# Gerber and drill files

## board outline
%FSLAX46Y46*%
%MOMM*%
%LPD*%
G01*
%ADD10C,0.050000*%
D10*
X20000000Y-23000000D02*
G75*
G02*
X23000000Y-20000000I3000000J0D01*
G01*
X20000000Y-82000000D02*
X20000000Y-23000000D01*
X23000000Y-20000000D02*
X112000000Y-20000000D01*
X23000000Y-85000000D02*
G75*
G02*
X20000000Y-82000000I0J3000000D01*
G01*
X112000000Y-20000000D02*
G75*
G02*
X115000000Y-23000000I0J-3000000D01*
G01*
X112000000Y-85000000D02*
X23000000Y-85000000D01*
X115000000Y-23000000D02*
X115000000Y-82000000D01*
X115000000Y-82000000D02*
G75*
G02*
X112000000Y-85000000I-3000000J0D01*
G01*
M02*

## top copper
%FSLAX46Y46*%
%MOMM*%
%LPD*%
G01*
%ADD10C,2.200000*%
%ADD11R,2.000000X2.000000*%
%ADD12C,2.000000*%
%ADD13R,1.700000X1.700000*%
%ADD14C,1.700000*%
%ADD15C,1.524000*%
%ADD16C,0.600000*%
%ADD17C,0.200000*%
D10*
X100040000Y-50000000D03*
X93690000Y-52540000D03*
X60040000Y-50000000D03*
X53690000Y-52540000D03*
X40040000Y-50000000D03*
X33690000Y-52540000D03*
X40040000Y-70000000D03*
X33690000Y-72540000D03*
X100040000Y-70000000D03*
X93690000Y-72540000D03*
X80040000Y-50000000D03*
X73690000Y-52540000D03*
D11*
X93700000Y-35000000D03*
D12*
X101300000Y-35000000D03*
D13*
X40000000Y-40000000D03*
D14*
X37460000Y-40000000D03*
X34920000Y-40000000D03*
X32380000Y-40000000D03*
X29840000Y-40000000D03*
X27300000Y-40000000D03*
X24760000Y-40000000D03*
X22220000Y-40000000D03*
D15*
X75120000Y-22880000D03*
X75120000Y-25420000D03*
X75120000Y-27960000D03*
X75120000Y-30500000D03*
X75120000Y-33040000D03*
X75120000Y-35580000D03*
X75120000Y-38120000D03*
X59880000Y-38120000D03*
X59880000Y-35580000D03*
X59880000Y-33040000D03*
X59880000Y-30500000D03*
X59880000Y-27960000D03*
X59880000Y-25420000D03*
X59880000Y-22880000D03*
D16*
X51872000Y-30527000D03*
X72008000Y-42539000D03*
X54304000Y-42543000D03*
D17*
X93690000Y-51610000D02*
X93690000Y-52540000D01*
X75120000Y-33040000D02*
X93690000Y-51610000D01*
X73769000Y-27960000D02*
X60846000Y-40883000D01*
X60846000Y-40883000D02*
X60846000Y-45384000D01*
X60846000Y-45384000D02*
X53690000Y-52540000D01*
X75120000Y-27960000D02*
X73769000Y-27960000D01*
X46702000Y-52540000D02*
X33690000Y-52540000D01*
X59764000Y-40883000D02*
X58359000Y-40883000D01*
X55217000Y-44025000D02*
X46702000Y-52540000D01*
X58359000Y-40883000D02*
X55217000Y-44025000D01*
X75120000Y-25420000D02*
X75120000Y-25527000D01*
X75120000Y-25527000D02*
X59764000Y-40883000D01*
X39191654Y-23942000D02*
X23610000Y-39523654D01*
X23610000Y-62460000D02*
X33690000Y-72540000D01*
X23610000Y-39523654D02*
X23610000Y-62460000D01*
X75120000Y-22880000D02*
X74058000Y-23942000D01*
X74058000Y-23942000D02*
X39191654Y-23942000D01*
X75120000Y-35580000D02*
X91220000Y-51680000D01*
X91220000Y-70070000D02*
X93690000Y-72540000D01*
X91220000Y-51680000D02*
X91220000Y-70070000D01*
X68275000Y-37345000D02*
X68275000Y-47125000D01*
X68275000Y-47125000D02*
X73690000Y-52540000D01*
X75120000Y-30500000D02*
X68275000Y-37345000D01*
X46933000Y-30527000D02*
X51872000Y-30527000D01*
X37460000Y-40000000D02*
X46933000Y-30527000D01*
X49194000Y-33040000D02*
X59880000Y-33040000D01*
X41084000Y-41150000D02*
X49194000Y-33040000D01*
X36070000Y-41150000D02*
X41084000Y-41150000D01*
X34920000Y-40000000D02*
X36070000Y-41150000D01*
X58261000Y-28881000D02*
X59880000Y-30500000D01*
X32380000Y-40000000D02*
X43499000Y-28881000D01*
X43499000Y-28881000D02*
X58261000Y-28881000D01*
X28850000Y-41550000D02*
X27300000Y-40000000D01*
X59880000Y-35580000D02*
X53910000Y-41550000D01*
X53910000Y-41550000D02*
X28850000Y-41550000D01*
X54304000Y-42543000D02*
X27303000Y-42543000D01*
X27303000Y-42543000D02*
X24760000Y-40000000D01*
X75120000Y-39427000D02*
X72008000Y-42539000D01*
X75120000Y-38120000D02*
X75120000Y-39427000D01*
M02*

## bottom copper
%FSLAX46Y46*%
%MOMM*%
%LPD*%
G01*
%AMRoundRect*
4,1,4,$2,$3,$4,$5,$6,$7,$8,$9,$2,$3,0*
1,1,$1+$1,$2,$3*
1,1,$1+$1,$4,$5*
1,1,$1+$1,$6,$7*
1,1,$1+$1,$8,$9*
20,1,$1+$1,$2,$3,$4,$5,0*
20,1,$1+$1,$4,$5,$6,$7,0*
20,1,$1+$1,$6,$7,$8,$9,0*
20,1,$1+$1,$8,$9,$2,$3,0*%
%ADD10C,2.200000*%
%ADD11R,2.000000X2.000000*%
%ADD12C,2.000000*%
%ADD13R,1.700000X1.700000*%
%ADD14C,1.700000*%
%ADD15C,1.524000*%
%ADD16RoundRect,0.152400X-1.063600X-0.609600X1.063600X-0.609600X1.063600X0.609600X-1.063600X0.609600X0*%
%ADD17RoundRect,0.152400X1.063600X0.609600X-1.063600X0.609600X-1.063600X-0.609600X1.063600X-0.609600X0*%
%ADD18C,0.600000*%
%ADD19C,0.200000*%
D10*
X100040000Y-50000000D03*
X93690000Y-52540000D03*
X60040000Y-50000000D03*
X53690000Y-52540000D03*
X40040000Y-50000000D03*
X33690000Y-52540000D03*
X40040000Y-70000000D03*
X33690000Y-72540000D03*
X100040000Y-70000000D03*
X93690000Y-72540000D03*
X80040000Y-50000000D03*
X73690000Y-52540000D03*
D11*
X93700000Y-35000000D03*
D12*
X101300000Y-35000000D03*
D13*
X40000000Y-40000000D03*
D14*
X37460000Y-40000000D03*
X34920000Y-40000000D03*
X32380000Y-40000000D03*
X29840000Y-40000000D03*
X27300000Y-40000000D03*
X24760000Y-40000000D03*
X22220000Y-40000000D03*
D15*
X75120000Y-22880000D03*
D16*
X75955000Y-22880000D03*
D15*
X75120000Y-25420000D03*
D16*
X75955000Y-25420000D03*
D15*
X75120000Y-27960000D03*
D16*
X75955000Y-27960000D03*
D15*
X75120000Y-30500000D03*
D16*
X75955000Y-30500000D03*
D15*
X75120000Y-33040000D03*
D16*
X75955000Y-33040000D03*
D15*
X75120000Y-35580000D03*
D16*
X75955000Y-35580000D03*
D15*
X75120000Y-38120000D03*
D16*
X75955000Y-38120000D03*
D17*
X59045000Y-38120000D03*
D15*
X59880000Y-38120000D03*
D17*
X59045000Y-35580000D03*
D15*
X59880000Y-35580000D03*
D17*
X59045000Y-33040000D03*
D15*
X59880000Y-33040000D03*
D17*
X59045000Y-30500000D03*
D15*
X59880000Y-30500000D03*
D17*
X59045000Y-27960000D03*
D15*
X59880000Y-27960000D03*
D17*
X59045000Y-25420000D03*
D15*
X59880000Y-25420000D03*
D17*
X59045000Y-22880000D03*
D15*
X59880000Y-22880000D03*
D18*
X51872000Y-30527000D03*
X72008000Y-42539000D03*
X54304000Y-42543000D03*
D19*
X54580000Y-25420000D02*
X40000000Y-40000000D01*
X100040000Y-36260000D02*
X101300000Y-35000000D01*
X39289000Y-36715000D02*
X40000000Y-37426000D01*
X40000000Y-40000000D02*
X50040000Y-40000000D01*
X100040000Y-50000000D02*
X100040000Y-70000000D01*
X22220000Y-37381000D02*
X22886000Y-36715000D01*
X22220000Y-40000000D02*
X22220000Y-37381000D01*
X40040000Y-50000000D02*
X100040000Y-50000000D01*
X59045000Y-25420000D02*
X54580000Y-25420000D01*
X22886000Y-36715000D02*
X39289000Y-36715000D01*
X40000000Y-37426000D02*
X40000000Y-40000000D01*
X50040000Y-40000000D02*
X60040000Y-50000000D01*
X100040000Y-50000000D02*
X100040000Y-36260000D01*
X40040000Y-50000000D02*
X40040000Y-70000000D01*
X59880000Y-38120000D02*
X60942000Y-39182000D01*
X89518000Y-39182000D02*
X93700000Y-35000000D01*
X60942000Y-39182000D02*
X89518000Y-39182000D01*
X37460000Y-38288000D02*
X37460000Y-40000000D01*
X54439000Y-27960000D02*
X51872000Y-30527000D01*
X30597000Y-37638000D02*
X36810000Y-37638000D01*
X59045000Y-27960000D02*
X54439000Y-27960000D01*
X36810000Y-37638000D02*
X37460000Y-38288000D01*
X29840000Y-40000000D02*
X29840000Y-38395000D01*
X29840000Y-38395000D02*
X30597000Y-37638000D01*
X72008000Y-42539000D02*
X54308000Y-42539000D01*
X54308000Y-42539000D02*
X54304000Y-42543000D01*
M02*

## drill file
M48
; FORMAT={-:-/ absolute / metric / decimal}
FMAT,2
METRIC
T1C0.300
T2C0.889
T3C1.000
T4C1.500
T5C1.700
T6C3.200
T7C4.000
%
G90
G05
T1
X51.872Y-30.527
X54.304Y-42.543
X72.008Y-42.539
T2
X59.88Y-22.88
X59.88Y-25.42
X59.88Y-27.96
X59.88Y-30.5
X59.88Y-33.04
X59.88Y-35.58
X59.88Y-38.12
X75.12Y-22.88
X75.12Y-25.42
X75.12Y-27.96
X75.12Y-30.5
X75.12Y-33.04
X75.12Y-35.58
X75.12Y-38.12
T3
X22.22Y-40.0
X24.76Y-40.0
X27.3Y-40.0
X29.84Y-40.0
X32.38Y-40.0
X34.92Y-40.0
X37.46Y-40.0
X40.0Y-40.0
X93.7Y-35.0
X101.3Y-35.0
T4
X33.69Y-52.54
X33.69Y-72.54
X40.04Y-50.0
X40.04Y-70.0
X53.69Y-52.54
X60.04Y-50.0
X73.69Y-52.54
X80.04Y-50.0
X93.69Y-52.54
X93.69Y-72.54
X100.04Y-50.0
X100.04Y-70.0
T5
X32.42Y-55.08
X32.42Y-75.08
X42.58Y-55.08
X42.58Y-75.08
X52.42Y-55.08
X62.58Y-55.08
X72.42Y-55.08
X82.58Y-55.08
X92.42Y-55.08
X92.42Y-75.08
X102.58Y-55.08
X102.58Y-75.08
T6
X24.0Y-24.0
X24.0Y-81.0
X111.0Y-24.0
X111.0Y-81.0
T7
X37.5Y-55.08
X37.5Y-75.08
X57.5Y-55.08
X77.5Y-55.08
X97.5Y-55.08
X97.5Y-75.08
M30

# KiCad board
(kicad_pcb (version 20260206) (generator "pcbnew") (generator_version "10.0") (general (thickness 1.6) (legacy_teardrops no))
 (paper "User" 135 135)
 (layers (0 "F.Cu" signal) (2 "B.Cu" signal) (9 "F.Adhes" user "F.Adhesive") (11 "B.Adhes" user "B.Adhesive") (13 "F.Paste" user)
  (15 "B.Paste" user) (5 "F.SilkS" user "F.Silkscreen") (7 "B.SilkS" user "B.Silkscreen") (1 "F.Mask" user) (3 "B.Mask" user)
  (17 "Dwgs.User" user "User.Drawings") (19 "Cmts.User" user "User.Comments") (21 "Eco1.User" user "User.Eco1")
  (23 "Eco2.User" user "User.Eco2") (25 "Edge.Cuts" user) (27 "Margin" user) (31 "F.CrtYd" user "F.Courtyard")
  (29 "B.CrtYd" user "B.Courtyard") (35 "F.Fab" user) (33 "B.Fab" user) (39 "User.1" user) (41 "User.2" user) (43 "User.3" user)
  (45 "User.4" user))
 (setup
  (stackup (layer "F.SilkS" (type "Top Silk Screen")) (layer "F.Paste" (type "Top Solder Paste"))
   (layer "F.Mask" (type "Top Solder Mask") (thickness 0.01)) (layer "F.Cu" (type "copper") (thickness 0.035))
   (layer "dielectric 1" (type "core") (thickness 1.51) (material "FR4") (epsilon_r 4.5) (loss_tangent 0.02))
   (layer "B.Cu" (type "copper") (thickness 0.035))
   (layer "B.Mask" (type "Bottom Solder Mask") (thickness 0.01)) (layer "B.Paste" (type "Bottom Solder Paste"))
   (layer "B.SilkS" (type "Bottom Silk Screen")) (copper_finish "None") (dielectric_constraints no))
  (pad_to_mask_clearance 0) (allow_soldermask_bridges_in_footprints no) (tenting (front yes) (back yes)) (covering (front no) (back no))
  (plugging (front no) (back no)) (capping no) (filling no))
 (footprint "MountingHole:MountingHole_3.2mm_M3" (layer "F.Cu") (at 24 81)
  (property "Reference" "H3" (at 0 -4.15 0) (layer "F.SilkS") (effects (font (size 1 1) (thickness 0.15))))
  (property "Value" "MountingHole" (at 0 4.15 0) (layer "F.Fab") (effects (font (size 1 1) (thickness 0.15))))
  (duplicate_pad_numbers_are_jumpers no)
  (pad "" np_thru_hole circle (at 0 0) (size 3.2 3.2) (drill 3.2) (layers "*.Cu" "*.Mask")))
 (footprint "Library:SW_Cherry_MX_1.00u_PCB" (layer "F.Cu") (at 100.04 50)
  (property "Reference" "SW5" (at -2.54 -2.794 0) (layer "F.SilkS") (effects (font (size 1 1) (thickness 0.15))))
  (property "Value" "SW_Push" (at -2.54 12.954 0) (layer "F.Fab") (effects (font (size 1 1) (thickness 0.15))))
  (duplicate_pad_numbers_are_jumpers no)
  (pad "" np_thru_hole circle (at -7.62 5.08) (size 1.7 1.7) (drill 1.7) (layers "*.Cu" "*.Mask"))
  (pad "" np_thru_hole circle (at -2.54 5.08) (size 4 4) (drill 4) (layers "*.Cu" "*.Mask"))
  (pad "" np_thru_hole circle (at 2.54 5.08) (size 1.7 1.7) (drill 1.7) (layers "*.Cu" "*.Mask"))
  (pad "1" thru_hole circle (at 0 0) (size 2.2 2.2) (drill 1.5) (layers "*.Cu" "*.Mask") (remove_unused_layers no) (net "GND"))
  (pad "2" thru_hole circle (at -6.35 2.54) (size 2.2 2.2) (drill 1.5) (layers "*.Cu" "*.Mask") (remove_unused_layers no)
   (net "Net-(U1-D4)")))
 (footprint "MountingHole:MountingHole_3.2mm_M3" (layer "F.Cu") (at 111 81)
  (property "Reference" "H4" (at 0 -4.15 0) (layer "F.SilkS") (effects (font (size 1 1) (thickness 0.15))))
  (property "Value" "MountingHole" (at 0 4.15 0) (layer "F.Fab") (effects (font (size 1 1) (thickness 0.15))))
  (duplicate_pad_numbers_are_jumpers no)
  (pad "" np_thru_hole circle (at 0 0) (size 3.2 3.2) (drill 3.2) (layers "*.Cu" "*.Mask")))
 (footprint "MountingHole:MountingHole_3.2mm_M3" (layer "F.Cu") (at 111 24 180)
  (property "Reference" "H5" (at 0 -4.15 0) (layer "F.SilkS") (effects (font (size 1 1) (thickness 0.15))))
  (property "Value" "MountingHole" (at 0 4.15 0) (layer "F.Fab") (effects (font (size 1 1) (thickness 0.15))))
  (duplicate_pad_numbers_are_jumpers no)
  (pad "" np_thru_hole circle (at 0 0 180) (size 3.2 3.2) (drill 3.2) (layers "*.Cu" "*.Mask")))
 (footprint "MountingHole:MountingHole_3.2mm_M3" (layer "F.Cu") (at 24 24 180)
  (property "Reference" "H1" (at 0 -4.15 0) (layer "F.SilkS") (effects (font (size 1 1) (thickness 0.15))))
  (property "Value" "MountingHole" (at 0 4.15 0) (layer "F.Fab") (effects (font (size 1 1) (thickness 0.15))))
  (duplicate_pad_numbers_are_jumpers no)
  (pad "" np_thru_hole circle (at 0 0 180) (size 3.2 3.2) (drill 3.2) (layers "*.Cu" "*.Mask")))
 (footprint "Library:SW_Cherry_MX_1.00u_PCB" (layer "F.Cu") (at 60.04 50)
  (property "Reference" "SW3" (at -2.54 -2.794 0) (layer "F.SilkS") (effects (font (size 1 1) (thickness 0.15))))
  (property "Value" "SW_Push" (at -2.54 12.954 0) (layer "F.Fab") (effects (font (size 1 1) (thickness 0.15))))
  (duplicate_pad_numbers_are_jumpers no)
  (pad "" np_thru_hole circle (at -7.62 5.08) (size 1.7 1.7) (drill 1.7) (layers "*.Cu" "*.Mask"))
  (pad "" np_thru_hole circle (at -2.54 5.08) (size 4 4) (drill 4) (layers "*.Cu" "*.Mask"))
  (pad "" np_thru_hole circle (at 2.54 5.08) (size 1.7 1.7) (drill 1.7) (layers "*.Cu" "*.Mask"))
  (pad "1" thru_hole circle (at 0 0) (size 2.2 2.2) (drill 1.5) (layers "*.Cu" "*.Mask") (remove_unused_layers no) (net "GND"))
  (pad "2" thru_hole circle (at -6.35 2.54) (size 2.2 2.2) (drill 1.5) (layers "*.Cu" "*.Mask") (remove_unused_layers no)
   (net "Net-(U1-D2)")))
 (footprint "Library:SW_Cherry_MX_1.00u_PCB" (layer "F.Cu") (at 40.04 50)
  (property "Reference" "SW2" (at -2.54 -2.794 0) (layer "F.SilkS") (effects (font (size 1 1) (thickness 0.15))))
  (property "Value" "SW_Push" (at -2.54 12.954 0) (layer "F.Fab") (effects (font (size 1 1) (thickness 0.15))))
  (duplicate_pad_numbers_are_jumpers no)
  (pad "" np_thru_hole circle (at -7.62 5.08) (size 1.7 1.7) (drill 1.7) (layers "*.Cu" "*.Mask"))
  (pad "" np_thru_hole circle (at -2.54 5.08) (size 4 4) (drill 4) (layers "*.Cu" "*.Mask"))
  (pad "" np_thru_hole circle (at 2.54 5.08) (size 1.7 1.7) (drill 1.7) (layers "*.Cu" "*.Mask"))
  (pad "1" thru_hole circle (at 0 0) (size 2.2 2.2) (drill 1.5) (layers "*.Cu" "*.Mask") (remove_unused_layers no) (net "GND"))
  (pad "2" thru_hole circle (at -6.35 2.54) (size 2.2 2.2) (drill 1.5) (layers "*.Cu" "*.Mask") (remove_unused_layers no)
   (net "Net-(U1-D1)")))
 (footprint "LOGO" (layer "F.Cu") (at 40 28)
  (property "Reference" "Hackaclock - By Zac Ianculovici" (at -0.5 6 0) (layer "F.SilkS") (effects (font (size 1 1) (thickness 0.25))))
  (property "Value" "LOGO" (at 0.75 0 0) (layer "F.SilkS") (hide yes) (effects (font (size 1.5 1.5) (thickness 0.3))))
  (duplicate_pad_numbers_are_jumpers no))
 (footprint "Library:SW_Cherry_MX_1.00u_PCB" (layer "F.Cu") (at 40.04 70)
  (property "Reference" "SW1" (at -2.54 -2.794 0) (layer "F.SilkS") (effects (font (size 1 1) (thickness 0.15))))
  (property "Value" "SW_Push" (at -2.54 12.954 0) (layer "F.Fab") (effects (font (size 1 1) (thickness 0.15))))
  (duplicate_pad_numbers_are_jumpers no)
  (pad "" np_thru_hole circle (at -7.62 5.08) (size 1.7 1.7) (drill 1.7) (layers "*.Cu" "*.Mask"))
  (pad "" np_thru_hole circle (at -2.54 5.08) (size 4 4) (drill 4) (layers "*.Cu" "*.Mask"))
  (pad "" np_thru_hole circle (at 2.54 5.08) (size 1.7 1.7) (drill 1.7) (layers "*.Cu" "*.Mask"))
  (pad "1" thru_hole circle (at 0 0) (size 2.2 2.2) (drill 1.5) (layers "*.Cu" "*.Mask") (remove_unused_layers no) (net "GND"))
  (pad "2" thru_hole circle (at -6.35 2.54) (size 2.2 2.2) (drill 1.5) (layers "*.Cu" "*.Mask") (remove_unused_layers no)
   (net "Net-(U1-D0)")))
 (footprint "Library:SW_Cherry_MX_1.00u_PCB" (layer "F.Cu") (at 100.04 70)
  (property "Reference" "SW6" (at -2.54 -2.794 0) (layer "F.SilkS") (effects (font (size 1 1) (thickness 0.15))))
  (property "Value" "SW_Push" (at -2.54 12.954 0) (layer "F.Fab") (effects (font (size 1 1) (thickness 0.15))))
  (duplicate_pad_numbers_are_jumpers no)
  (pad "" np_thru_hole circle (at -7.62 5.08) (size 1.7 1.7) (drill 1.7) (layers "*.Cu" "*.Mask"))
  (pad "" np_thru_hole circle (at -2.54 5.08) (size 4 4) (drill 4) (layers "*.Cu" "*.Mask"))
  (pad "" np_thru_hole circle (at 2.54 5.08) (size 1.7 1.7) (drill 1.7) (layers "*.Cu" "*.Mask"))
  (pad "1" thru_hole circle (at 0 0) (size 2.2 2.2) (drill 1.5) (layers "*.Cu" "*.Mask") (remove_unused_layers no) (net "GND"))
  (pad "2" thru_hole circle (at -6.35 2.54) (size 2.2 2.2) (drill 1.5) (layers "*.Cu" "*.Mask") (remove_unused_layers no)
   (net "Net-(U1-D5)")))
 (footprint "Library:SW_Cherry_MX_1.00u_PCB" (layer "F.Cu") (at 80.04 50)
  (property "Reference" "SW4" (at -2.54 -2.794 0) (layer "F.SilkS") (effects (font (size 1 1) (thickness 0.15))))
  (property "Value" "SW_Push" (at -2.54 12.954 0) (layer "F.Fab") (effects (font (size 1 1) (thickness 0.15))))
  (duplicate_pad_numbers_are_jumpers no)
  (pad "" np_thru_hole circle (at -7.62 5.08) (size 1.7 1.7) (drill 1.7) (layers "*.Cu" "*.Mask"))
  (pad "" np_thru_hole circle (at -2.54 5.08) (size 4 4) (drill 4) (layers "*.Cu" "*.Mask"))
  (pad "" np_thru_hole circle (at 2.54 5.08) (size 1.7 1.7) (drill 1.7) (layers "*.Cu" "*.Mask"))
  (pad "1" thru_hole circle (at 0 0) (size 2.2 2.2) (drill 1.5) (layers "*.Cu" "*.Mask") (remove_unused_layers no) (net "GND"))
  (pad "2" thru_hole circle (at -6.35 2.54) (size 2.2 2.2) (drill 1.5) (layers "*.Cu" "*.Mask") (remove_unused_layers no)
   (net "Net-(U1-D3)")))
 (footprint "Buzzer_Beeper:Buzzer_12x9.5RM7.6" (layer "B.Cu") (at 93.7 35)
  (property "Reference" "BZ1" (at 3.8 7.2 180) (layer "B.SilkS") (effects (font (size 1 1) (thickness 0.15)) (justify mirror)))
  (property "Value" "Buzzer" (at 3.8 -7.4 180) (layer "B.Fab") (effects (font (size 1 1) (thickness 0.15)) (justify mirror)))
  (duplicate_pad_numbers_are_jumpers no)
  (pad "1" thru_hole rect (at 0 0) (size 2 2) (drill 1) (layers "*.Cu" "*.Mask") (remove_unused_layers no) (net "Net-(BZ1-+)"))
  (pad "2" thru_hole circle (at 7.6 0) (size 2 2) (drill 1) (layers "*.Cu" "*.Mask") (remove_unused_layers no) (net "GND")))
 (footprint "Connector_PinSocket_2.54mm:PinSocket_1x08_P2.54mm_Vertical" (layer "B.Cu") (at 40 40 90)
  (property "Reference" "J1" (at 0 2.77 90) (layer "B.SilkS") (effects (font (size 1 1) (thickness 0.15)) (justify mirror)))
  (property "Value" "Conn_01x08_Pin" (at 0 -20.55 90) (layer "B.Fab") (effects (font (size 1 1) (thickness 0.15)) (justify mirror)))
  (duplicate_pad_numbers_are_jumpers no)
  (pad "1" thru_hole rect (at 0 0 90) (size 1.7 1.7) (drill 1) (layers "*.Cu" "*.Mask") (remove_unused_layers no) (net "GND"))
  (pad "2" thru_hole circle (at 0 -2.54 90) (size 1.7 1.7) (drill 1) (layers "*.Cu" "*.Mask") (remove_unused_layers no) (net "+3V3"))
  (pad "3" thru_hole circle (at 0 -5.08 90) (size 1.7 1.7) (drill 1) (layers "*.Cu" "*.Mask") (remove_unused_layers no) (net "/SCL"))
  (pad "4" thru_hole circle (at 0 -7.62 90) (size 1.7 1.7) (drill 1) (layers "*.Cu" "*.Mask") (remove_unused_layers no) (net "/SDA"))
  (pad "5" thru_hole circle (at 0 -10.16 90) (size 1.7 1.7) (drill 1) (layers "*.Cu" "*.Mask") (remove_unused_layers no) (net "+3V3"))
  (pad "6" thru_hole circle (at 0 -12.7 90) (size 1.7 1.7) (drill 1) (layers "*.Cu" "*.Mask") (remove_unused_layers no) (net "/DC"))
  (pad "7" thru_hole circle (at 0 -15.24 90) (size 1.7 1.7) (drill 1) (layers "*.Cu" "*.Mask") (remove_unused_layers no) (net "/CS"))
  (pad "8" thru_hole circle (at 0 -17.78 90) (size 1.7 1.7) (drill 1) (layers "*.Cu" "*.Mask") (remove_unused_layers no) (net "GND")))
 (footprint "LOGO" (layer "B.Cu") (at 40 28 180)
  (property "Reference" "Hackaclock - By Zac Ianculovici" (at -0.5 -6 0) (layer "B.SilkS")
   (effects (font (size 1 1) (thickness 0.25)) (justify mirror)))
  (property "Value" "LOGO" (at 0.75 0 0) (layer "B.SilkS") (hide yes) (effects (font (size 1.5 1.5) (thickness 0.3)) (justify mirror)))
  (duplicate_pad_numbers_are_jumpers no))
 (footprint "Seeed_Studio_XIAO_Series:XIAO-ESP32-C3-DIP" (layer "B.Cu") (at 67.5 30.5 90)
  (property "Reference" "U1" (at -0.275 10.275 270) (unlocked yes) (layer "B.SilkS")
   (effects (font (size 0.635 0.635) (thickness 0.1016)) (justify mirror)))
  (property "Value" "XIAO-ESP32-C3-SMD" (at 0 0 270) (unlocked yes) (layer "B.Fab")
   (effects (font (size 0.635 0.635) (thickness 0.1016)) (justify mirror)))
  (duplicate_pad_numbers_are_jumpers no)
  (pad "1" thru_hole circle (at 7.62 7.62) (size 1.524 1.524) (drill 0.889) (layers "*.Cu" "*.Mask") (remove_unused_layers no)
   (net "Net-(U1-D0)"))
  (pad "1" smd roundrect (at 7.62 8.455) (size 2.432 1.524) (layers "B.Cu" "B.Mask") (roundrect_rratio 0.1) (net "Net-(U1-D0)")
   (thermal_bridge_angle 45))
  (pad "2" thru_hole circle (at 5.08 7.62) (size 1.524 1.524) (drill 0.889) (layers "*.Cu" "*.Mask") (remove_unused_layers no)
   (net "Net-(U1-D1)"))
  (pad "2" smd roundrect (at 5.08 8.455) (size 2.432 1.524) (layers "B.Cu" "B.Mask") (roundrect_rratio 0.1) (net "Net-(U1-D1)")
   (thermal_bridge_angle 45))
  (pad "3" thru_hole circle (at 2.54 7.62) (size 1.524 1.524) (drill 0.889) (layers "*.Cu" "*.Mask") (remove_unused_layers no)
   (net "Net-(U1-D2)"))
  (pad "3" smd roundrect (at 2.54 8.455) (size 2.432 1.524) (layers "B.Cu" "B.Mask") (roundrect_rratio 0.1) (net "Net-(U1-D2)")
   (thermal_bridge_angle 45))
  (pad "4" thru_hole circle (at 0 7.62) (size 1.524 1.524) (drill 0.889) (layers "*.Cu" "*.Mask") (remove_unused_layers no)
   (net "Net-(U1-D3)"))
  (pad "4" smd roundrect (at 0 8.455) (size 2.432 1.524) (layers "B.Cu" "B.Mask") (roundrect_rratio 0.1) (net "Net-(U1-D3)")
   (thermal_bridge_angle 45))
  (pad "5" thru_hole circle (at -2.54 7.62) (size 1.524 1.524) (drill 0.889) (layers "*.Cu" "*.Mask") (remove_unused_layers no)
   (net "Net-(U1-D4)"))
  (pad "5" smd roundrect (at -2.54 8.455) (size 2.432 1.524) (layers "B.Cu" "B.Mask") (roundrect_rratio 0.1) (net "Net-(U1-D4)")
   (thermal_bridge_angle 45))
  (pad "6" thru_hole circle (at -5.08 7.62) (size 1.524 1.524) (drill 0.889) (layers "*.Cu" "*.Mask") (remove_unused_layers no)
   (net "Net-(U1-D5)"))
  (pad "6" smd roundrect (at -5.08 8.455) (size 2.432 1.524) (layers "B.Cu" "B.Mask") (roundrect_rratio 0.1) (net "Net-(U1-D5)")
   (thermal_bridge_angle 45))
  (pad "7" thru_hole circle (at -7.62 7.62) (size 1.524 1.524) (drill 0.889) (layers "*.Cu" "*.Mask") (remove_unused_layers no) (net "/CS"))
  (pad "7" smd roundrect (at -7.62 8.455) (size 2.432 1.524) (layers "B.Cu" "B.Mask") (roundrect_rratio 0.1) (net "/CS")
   (thermal_bridge_angle 45))
  (pad "8" smd roundrect (at -7.62 -8.455 180) (size 2.432 1.524) (layers "B.Cu" "B.Mask") (roundrect_rratio 0.1) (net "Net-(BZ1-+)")
   (thermal_bridge_angle 45))
  (pad "8" thru_hole circle (at -7.62 -7.62 180) (size 1.524 1.524) (drill 0.889) (layers "*.Cu" "*.Mask") (remove_unused_layers no)
   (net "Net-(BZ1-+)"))
  (pad "9" smd roundrect (at -5.08 -8.455 180) (size 2.432 1.524) (layers "B.Cu" "B.Mask") (roundrect_rratio 0.1) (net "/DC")
   (thermal_bridge_angle 45))
  (pad "9" thru_hole circle (at -5.08 -7.62 180) (size 1.524 1.524) (drill 0.889) (layers "*.Cu" "*.Mask") (remove_unused_layers no)
   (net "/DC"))
  (pad "10" smd roundrect (at -2.54 -8.455 180) (size 2.432 1.524) (layers "B.Cu" "B.Mask") (roundrect_rratio 0.1) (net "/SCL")
   (thermal_bridge_angle 45))
  (pad "10" thru_hole circle (at -2.54 -7.62 180) (size 1.524 1.524) (drill 0.889) (layers "*.Cu" "*.Mask") (remove_unused_layers no)
   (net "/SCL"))
  (pad "11" smd roundrect (at 0 -8.455 180) (size 2.432 1.524) (layers "B.Cu" "B.Mask") (roundrect_rratio 0.1) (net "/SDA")
   (thermal_bridge_angle 45))
  (pad "11" thru_hole circle (at 0 -7.62 180) (size 1.524 1.524) (drill 0.889) (layers "*.Cu" "*.Mask") (remove_unused_layers no)
   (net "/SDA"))
  (pad "12" smd roundrect (at 2.54 -8.455 180) (size 2.432 1.524) (layers "B.Cu" "B.Mask") (roundrect_rratio 0.1) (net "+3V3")
   (thermal_bridge_angle 45))
  (pad "12" thru_hole circle (at 2.54 -7.62 180) (size 1.524 1.524) (drill 0.889) (layers "*.Cu" "*.Mask") (remove_unused_layers no)
   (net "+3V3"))
  (pad "13" smd roundrect (at 5.08 -8.455 180) (size 2.432 1.524) (layers "B.Cu" "B.Mask") (roundrect_rratio 0.1) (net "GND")
   (thermal_bridge_angle 45))
  (pad "13" thru_hole circle (at 5.08 -7.62 180) (size 1.524 1.524) (drill 0.889) (layers "*.Cu" "*.Mask") (remove_unused_layers no)
   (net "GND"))
  (pad "14" smd roundrect (at 7.62 -8.455 180) (size 2.432 1.524) (layers "B.Cu" "B.Mask") (roundrect_rratio 0.1)
   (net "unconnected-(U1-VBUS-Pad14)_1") (thermal_bridge_angle 45))
  (pad "14" thru_hole circle (at 7.62 -7.62 180) (size 1.524 1.524) (drill 0.889) (layers "*.Cu" "*.Mask") (remove_unused_layers no)
   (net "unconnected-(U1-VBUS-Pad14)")))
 (gr_arc (start 20 23) (mid 20.87868 20.87868) (end 23 20) (stroke (width 0.05) (type default)) (layer "Edge.Cuts"))
 (gr_line (start 20 82) (end 20 23) (stroke (width 0.05) (type default)) (layer "Edge.Cuts"))
 (gr_line (start 23 20) (end 112 20) (stroke (width 0.05) (type default)) (layer "Edge.Cuts"))
 (gr_arc (start 23 85) (mid 20.87868 84.12132) (end 20 82) (stroke (width 0.05) (type default)) (layer "Edge.Cuts"))
 (gr_arc (start 112 20) (mid 114.12132 20.87868) (end 115 23) (stroke (width 0.05) (type default)) (layer "Edge.Cuts"))
 (gr_line (start 112 85) (end 23 85) (stroke (width 0.05) (type default)) (layer "Edge.Cuts"))
 (gr_line (start 115 23) (end 115 82) (stroke (width 0.05) (type default)) (layer "Edge.Cuts"))
 (gr_arc (start 115 82) (mid 114.12132 84.12132) (end 112 85) (stroke (width 0.05) (type default)) (layer "Edge.Cuts"))
 (segment (start 54.58 25.42) (end 40 40) (width 0.2) (layer "B.Cu") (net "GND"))
 (segment (start 100.04 36.26) (end 101.3 35) (width 0.2) (layer "B.Cu") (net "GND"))
 (segment (start 39.289 36.715) (end 40 37.426) (width 0.2) (layer "B.Cu") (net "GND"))
 (segment (start 40 40) (end 50.04 40) (width 0.2) (layer "B.Cu") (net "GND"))
 (segment (start 100.04 50) (end 100.04 70) (width 0.2) (layer "B.Cu") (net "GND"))
 (segment (start 22.22 37.381) (end 22.886 36.715) (width 0.2) (layer "B.Cu") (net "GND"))
 (segment (start 22.22 40) (end 22.22 37.381) (width 0.2) (layer "B.Cu") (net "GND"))
 (segment (start 40.04 50) (end 100.04 50) (width 0.2) (layer "B.Cu") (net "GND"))
 (segment (start 59.045 25.42) (end 54.58 25.42) (width 0.2) (layer "B.Cu") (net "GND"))
 (segment (start 22.886 36.715) (end 39.289 36.715) (width 0.2) (layer "B.Cu") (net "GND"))
 (segment (start 40 37.426) (end 40 40) (width 0.2) (layer "B.Cu") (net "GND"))
 (segment (start 50.04 40) (end 60.04 50) (width 0.2) (layer "B.Cu") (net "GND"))
 (segment (start 100.04 50) (end 100.04 36.26) (width 0.2) (layer "B.Cu") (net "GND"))
 (segment (start 40.04 50) (end 40.04 70) (width 0.2) (layer "B.Cu") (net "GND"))
 (segment (start 93.69 51.61) (end 93.69 52.54) (width 0.2) (layer "F.Cu") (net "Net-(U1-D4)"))
 (segment (start 75.12 33.04) (end 93.69 51.61) (width 0.2) (layer "F.Cu") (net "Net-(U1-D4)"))
 (segment (start 73.769 27.96) (end 60.846 40.883) (width 0.2) (layer "F.Cu") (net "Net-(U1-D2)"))
 (segment (start 60.846 40.883) (end 60.846 45.384) (width 0.2) (layer "F.Cu") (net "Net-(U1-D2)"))
 (segment (start 60.846 45.384) (end 53.69 52.54) (width 0.2) (layer "F.Cu") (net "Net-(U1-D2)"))
 (segment (start 75.12 27.96) (end 73.769 27.96) (width 0.2) (layer "F.Cu") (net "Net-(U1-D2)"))
 (segment (start 46.702 52.54) (end 33.69 52.54) (width 0.2) (layer "F.Cu") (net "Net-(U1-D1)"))
 (segment (start 59.764 40.883) (end 58.359 40.883) (width 0.2) (layer "F.Cu") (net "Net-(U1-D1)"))
 (segment (start 55.217 44.025) (end 46.702 52.54) (width 0.2) (layer "F.Cu") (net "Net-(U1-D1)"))
 (segment (start 58.359 40.883) (end 55.217 44.025) (width 0.2) (layer "F.Cu") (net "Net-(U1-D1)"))
 (segment (start 75.12 25.42) (end 75.12 25.527) (width 0.2) (layer "F.Cu") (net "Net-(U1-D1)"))
 (segment (start 75.12 25.527) (end 59.764 40.883) (width 0.2) (layer "F.Cu") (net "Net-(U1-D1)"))
 (segment (start 39.191654 23.942) (end 23.61 39.523654) (width 0.2) (layer "F.Cu") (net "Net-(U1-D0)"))
 (segment (start 23.61 62.46) (end 33.69 72.54) (width 0.2) (layer "F.Cu") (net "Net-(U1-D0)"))
 (segment (start 23.61 39.523654) (end 23.61 62.46) (width 0.2) (layer "F.Cu") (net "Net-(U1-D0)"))
 (segment (start 75.12 22.88) (end 74.058 23.942) (width 0.2) (layer "F.Cu") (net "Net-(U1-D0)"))
 (segment (start 74.058 23.942) (end 39.191654 23.942) (width 0.2) (layer "F.Cu") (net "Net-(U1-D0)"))
 (segment (start 75.12 35.58) (end 91.22 51.68) (width 0.2) (layer "F.Cu") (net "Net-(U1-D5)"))
 (segment (start 91.22 70.07) (end 93.69 72.54) (width 0.2) (layer "F.Cu") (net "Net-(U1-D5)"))
 (segment (start 91.22 51.68) (end 91.22 70.07) (width 0.2) (layer "F.Cu") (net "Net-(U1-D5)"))
 (segment (start 68.275 37.345) (end 68.275 47.125) (width 0.2) (layer "F.Cu") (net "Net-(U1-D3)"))
 (segment (start 68.275 47.125) (end 73.69 52.54) (width 0.2) (layer "F.Cu") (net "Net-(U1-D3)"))
 (segment (start 75.12 30.5) (end 68.275 37.345) (width 0.2) (layer "F.Cu") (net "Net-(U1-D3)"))
 (segment (start 59.88 38.12) (end 60.942 39.182) (width 0.2) (layer "B.Cu") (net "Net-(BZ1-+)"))
 (segment (start 89.518 39.182) (end 93.7 35) (width 0.2) (layer "B.Cu") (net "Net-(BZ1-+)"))
 (segment (start 60.942 39.182) (end 89.518 39.182) (width 0.2) (layer "B.Cu") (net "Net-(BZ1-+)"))
 (segment (start 46.933 30.527) (end 51.872 30.527) (width 0.2) (layer "F.Cu") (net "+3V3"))
 (segment (start 37.46 40) (end 46.933 30.527) (width 0.2) (layer "F.Cu") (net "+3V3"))
 (via (at 51.872 30.527) (size 0.6) (drill 0.3) (layers "F.Cu" "B.Cu") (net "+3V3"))
 (segment (start 37.46 38.288) (end 37.46 40) (width 0.2) (layer "B.Cu") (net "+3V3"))
 (segment (start 54.439 27.96) (end 51.872 30.527) (width 0.2) (layer "B.Cu") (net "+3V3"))
 (segment (start 30.597 37.638) (end 36.81 37.638) (width 0.2) (layer "B.Cu") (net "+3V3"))
 (segment (start 59.045 27.96) (end 54.439 27.96) (width 0.2) (layer "B.Cu") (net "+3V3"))
 (segment (start 36.81 37.638) (end 37.46 38.288) (width 0.2) (layer "B.Cu") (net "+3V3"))
 (segment (start 29.84 40) (end 29.84 38.395) (width 0.2) (layer "B.Cu") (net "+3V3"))
 (segment (start 29.84 38.395) (end 30.597 37.638) (width 0.2) (layer "B.Cu") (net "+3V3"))
 (segment (start 49.194 33.04) (end 59.88 33.04) (width 0.2) (layer "F.Cu") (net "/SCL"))
 (segment (start 41.084 41.15) (end 49.194 33.04) (width 0.2) (layer "F.Cu") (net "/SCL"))
 (segment (start 36.07 41.15) (end 41.084 41.15) (width 0.2) (layer "F.Cu") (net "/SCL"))
 (segment (start 34.92 40) (end 36.07 41.15) (width 0.2) (layer "F.Cu") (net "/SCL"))
 (segment (start 58.261 28.881) (end 59.88 30.5) (width 0.2) (layer "F.Cu") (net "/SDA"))
 (segment (start 32.38 40) (end 43.499 28.881) (width 0.2) (layer "F.Cu") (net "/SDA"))
 (segment (start 43.499 28.881) (end 58.261 28.881) (width 0.2) (layer "F.Cu") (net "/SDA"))
 (segment (start 28.85 41.55) (end 27.3 40) (width 0.2) (layer "F.Cu") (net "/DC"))
 (segment (start 59.88 35.58) (end 53.91 41.55) (width 0.2) (layer "F.Cu") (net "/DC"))
 (segment (start 53.91 41.55) (end 28.85 41.55) (width 0.2) (layer "F.Cu") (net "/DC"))
 (segment (start 54.304 42.543) (end 27.303 42.543) (width 0.2) (layer "F.Cu") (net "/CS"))
 (segment (start 27.303 42.543) (end 24.76 40) (width 0.2) (layer "F.Cu") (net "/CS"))
 (segment (start 75.12 39.427) (end 72.008 42.539) (width 0.2) (layer "F.Cu") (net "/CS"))
 (segment (start 75.12 38.12) (end 75.12 39.427) (width 0.2) (layer "F.Cu") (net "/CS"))
 (via (at 72.008 42.539) (size 0.6) (drill 0.3) (layers "F.Cu" "B.Cu") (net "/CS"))
 (via (at 54.304 42.543) (size 0.6) (drill 0.3) (layers "F.Cu" "B.Cu") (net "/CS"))
 (segment (start 72.008 42.539) (end 54.308 42.539) (width 0.2) (layer "B.Cu") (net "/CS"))
 (segment (start 54.308 42.539) (end 54.304 42.543) (width 0.2) (layer "B.Cu") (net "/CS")))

